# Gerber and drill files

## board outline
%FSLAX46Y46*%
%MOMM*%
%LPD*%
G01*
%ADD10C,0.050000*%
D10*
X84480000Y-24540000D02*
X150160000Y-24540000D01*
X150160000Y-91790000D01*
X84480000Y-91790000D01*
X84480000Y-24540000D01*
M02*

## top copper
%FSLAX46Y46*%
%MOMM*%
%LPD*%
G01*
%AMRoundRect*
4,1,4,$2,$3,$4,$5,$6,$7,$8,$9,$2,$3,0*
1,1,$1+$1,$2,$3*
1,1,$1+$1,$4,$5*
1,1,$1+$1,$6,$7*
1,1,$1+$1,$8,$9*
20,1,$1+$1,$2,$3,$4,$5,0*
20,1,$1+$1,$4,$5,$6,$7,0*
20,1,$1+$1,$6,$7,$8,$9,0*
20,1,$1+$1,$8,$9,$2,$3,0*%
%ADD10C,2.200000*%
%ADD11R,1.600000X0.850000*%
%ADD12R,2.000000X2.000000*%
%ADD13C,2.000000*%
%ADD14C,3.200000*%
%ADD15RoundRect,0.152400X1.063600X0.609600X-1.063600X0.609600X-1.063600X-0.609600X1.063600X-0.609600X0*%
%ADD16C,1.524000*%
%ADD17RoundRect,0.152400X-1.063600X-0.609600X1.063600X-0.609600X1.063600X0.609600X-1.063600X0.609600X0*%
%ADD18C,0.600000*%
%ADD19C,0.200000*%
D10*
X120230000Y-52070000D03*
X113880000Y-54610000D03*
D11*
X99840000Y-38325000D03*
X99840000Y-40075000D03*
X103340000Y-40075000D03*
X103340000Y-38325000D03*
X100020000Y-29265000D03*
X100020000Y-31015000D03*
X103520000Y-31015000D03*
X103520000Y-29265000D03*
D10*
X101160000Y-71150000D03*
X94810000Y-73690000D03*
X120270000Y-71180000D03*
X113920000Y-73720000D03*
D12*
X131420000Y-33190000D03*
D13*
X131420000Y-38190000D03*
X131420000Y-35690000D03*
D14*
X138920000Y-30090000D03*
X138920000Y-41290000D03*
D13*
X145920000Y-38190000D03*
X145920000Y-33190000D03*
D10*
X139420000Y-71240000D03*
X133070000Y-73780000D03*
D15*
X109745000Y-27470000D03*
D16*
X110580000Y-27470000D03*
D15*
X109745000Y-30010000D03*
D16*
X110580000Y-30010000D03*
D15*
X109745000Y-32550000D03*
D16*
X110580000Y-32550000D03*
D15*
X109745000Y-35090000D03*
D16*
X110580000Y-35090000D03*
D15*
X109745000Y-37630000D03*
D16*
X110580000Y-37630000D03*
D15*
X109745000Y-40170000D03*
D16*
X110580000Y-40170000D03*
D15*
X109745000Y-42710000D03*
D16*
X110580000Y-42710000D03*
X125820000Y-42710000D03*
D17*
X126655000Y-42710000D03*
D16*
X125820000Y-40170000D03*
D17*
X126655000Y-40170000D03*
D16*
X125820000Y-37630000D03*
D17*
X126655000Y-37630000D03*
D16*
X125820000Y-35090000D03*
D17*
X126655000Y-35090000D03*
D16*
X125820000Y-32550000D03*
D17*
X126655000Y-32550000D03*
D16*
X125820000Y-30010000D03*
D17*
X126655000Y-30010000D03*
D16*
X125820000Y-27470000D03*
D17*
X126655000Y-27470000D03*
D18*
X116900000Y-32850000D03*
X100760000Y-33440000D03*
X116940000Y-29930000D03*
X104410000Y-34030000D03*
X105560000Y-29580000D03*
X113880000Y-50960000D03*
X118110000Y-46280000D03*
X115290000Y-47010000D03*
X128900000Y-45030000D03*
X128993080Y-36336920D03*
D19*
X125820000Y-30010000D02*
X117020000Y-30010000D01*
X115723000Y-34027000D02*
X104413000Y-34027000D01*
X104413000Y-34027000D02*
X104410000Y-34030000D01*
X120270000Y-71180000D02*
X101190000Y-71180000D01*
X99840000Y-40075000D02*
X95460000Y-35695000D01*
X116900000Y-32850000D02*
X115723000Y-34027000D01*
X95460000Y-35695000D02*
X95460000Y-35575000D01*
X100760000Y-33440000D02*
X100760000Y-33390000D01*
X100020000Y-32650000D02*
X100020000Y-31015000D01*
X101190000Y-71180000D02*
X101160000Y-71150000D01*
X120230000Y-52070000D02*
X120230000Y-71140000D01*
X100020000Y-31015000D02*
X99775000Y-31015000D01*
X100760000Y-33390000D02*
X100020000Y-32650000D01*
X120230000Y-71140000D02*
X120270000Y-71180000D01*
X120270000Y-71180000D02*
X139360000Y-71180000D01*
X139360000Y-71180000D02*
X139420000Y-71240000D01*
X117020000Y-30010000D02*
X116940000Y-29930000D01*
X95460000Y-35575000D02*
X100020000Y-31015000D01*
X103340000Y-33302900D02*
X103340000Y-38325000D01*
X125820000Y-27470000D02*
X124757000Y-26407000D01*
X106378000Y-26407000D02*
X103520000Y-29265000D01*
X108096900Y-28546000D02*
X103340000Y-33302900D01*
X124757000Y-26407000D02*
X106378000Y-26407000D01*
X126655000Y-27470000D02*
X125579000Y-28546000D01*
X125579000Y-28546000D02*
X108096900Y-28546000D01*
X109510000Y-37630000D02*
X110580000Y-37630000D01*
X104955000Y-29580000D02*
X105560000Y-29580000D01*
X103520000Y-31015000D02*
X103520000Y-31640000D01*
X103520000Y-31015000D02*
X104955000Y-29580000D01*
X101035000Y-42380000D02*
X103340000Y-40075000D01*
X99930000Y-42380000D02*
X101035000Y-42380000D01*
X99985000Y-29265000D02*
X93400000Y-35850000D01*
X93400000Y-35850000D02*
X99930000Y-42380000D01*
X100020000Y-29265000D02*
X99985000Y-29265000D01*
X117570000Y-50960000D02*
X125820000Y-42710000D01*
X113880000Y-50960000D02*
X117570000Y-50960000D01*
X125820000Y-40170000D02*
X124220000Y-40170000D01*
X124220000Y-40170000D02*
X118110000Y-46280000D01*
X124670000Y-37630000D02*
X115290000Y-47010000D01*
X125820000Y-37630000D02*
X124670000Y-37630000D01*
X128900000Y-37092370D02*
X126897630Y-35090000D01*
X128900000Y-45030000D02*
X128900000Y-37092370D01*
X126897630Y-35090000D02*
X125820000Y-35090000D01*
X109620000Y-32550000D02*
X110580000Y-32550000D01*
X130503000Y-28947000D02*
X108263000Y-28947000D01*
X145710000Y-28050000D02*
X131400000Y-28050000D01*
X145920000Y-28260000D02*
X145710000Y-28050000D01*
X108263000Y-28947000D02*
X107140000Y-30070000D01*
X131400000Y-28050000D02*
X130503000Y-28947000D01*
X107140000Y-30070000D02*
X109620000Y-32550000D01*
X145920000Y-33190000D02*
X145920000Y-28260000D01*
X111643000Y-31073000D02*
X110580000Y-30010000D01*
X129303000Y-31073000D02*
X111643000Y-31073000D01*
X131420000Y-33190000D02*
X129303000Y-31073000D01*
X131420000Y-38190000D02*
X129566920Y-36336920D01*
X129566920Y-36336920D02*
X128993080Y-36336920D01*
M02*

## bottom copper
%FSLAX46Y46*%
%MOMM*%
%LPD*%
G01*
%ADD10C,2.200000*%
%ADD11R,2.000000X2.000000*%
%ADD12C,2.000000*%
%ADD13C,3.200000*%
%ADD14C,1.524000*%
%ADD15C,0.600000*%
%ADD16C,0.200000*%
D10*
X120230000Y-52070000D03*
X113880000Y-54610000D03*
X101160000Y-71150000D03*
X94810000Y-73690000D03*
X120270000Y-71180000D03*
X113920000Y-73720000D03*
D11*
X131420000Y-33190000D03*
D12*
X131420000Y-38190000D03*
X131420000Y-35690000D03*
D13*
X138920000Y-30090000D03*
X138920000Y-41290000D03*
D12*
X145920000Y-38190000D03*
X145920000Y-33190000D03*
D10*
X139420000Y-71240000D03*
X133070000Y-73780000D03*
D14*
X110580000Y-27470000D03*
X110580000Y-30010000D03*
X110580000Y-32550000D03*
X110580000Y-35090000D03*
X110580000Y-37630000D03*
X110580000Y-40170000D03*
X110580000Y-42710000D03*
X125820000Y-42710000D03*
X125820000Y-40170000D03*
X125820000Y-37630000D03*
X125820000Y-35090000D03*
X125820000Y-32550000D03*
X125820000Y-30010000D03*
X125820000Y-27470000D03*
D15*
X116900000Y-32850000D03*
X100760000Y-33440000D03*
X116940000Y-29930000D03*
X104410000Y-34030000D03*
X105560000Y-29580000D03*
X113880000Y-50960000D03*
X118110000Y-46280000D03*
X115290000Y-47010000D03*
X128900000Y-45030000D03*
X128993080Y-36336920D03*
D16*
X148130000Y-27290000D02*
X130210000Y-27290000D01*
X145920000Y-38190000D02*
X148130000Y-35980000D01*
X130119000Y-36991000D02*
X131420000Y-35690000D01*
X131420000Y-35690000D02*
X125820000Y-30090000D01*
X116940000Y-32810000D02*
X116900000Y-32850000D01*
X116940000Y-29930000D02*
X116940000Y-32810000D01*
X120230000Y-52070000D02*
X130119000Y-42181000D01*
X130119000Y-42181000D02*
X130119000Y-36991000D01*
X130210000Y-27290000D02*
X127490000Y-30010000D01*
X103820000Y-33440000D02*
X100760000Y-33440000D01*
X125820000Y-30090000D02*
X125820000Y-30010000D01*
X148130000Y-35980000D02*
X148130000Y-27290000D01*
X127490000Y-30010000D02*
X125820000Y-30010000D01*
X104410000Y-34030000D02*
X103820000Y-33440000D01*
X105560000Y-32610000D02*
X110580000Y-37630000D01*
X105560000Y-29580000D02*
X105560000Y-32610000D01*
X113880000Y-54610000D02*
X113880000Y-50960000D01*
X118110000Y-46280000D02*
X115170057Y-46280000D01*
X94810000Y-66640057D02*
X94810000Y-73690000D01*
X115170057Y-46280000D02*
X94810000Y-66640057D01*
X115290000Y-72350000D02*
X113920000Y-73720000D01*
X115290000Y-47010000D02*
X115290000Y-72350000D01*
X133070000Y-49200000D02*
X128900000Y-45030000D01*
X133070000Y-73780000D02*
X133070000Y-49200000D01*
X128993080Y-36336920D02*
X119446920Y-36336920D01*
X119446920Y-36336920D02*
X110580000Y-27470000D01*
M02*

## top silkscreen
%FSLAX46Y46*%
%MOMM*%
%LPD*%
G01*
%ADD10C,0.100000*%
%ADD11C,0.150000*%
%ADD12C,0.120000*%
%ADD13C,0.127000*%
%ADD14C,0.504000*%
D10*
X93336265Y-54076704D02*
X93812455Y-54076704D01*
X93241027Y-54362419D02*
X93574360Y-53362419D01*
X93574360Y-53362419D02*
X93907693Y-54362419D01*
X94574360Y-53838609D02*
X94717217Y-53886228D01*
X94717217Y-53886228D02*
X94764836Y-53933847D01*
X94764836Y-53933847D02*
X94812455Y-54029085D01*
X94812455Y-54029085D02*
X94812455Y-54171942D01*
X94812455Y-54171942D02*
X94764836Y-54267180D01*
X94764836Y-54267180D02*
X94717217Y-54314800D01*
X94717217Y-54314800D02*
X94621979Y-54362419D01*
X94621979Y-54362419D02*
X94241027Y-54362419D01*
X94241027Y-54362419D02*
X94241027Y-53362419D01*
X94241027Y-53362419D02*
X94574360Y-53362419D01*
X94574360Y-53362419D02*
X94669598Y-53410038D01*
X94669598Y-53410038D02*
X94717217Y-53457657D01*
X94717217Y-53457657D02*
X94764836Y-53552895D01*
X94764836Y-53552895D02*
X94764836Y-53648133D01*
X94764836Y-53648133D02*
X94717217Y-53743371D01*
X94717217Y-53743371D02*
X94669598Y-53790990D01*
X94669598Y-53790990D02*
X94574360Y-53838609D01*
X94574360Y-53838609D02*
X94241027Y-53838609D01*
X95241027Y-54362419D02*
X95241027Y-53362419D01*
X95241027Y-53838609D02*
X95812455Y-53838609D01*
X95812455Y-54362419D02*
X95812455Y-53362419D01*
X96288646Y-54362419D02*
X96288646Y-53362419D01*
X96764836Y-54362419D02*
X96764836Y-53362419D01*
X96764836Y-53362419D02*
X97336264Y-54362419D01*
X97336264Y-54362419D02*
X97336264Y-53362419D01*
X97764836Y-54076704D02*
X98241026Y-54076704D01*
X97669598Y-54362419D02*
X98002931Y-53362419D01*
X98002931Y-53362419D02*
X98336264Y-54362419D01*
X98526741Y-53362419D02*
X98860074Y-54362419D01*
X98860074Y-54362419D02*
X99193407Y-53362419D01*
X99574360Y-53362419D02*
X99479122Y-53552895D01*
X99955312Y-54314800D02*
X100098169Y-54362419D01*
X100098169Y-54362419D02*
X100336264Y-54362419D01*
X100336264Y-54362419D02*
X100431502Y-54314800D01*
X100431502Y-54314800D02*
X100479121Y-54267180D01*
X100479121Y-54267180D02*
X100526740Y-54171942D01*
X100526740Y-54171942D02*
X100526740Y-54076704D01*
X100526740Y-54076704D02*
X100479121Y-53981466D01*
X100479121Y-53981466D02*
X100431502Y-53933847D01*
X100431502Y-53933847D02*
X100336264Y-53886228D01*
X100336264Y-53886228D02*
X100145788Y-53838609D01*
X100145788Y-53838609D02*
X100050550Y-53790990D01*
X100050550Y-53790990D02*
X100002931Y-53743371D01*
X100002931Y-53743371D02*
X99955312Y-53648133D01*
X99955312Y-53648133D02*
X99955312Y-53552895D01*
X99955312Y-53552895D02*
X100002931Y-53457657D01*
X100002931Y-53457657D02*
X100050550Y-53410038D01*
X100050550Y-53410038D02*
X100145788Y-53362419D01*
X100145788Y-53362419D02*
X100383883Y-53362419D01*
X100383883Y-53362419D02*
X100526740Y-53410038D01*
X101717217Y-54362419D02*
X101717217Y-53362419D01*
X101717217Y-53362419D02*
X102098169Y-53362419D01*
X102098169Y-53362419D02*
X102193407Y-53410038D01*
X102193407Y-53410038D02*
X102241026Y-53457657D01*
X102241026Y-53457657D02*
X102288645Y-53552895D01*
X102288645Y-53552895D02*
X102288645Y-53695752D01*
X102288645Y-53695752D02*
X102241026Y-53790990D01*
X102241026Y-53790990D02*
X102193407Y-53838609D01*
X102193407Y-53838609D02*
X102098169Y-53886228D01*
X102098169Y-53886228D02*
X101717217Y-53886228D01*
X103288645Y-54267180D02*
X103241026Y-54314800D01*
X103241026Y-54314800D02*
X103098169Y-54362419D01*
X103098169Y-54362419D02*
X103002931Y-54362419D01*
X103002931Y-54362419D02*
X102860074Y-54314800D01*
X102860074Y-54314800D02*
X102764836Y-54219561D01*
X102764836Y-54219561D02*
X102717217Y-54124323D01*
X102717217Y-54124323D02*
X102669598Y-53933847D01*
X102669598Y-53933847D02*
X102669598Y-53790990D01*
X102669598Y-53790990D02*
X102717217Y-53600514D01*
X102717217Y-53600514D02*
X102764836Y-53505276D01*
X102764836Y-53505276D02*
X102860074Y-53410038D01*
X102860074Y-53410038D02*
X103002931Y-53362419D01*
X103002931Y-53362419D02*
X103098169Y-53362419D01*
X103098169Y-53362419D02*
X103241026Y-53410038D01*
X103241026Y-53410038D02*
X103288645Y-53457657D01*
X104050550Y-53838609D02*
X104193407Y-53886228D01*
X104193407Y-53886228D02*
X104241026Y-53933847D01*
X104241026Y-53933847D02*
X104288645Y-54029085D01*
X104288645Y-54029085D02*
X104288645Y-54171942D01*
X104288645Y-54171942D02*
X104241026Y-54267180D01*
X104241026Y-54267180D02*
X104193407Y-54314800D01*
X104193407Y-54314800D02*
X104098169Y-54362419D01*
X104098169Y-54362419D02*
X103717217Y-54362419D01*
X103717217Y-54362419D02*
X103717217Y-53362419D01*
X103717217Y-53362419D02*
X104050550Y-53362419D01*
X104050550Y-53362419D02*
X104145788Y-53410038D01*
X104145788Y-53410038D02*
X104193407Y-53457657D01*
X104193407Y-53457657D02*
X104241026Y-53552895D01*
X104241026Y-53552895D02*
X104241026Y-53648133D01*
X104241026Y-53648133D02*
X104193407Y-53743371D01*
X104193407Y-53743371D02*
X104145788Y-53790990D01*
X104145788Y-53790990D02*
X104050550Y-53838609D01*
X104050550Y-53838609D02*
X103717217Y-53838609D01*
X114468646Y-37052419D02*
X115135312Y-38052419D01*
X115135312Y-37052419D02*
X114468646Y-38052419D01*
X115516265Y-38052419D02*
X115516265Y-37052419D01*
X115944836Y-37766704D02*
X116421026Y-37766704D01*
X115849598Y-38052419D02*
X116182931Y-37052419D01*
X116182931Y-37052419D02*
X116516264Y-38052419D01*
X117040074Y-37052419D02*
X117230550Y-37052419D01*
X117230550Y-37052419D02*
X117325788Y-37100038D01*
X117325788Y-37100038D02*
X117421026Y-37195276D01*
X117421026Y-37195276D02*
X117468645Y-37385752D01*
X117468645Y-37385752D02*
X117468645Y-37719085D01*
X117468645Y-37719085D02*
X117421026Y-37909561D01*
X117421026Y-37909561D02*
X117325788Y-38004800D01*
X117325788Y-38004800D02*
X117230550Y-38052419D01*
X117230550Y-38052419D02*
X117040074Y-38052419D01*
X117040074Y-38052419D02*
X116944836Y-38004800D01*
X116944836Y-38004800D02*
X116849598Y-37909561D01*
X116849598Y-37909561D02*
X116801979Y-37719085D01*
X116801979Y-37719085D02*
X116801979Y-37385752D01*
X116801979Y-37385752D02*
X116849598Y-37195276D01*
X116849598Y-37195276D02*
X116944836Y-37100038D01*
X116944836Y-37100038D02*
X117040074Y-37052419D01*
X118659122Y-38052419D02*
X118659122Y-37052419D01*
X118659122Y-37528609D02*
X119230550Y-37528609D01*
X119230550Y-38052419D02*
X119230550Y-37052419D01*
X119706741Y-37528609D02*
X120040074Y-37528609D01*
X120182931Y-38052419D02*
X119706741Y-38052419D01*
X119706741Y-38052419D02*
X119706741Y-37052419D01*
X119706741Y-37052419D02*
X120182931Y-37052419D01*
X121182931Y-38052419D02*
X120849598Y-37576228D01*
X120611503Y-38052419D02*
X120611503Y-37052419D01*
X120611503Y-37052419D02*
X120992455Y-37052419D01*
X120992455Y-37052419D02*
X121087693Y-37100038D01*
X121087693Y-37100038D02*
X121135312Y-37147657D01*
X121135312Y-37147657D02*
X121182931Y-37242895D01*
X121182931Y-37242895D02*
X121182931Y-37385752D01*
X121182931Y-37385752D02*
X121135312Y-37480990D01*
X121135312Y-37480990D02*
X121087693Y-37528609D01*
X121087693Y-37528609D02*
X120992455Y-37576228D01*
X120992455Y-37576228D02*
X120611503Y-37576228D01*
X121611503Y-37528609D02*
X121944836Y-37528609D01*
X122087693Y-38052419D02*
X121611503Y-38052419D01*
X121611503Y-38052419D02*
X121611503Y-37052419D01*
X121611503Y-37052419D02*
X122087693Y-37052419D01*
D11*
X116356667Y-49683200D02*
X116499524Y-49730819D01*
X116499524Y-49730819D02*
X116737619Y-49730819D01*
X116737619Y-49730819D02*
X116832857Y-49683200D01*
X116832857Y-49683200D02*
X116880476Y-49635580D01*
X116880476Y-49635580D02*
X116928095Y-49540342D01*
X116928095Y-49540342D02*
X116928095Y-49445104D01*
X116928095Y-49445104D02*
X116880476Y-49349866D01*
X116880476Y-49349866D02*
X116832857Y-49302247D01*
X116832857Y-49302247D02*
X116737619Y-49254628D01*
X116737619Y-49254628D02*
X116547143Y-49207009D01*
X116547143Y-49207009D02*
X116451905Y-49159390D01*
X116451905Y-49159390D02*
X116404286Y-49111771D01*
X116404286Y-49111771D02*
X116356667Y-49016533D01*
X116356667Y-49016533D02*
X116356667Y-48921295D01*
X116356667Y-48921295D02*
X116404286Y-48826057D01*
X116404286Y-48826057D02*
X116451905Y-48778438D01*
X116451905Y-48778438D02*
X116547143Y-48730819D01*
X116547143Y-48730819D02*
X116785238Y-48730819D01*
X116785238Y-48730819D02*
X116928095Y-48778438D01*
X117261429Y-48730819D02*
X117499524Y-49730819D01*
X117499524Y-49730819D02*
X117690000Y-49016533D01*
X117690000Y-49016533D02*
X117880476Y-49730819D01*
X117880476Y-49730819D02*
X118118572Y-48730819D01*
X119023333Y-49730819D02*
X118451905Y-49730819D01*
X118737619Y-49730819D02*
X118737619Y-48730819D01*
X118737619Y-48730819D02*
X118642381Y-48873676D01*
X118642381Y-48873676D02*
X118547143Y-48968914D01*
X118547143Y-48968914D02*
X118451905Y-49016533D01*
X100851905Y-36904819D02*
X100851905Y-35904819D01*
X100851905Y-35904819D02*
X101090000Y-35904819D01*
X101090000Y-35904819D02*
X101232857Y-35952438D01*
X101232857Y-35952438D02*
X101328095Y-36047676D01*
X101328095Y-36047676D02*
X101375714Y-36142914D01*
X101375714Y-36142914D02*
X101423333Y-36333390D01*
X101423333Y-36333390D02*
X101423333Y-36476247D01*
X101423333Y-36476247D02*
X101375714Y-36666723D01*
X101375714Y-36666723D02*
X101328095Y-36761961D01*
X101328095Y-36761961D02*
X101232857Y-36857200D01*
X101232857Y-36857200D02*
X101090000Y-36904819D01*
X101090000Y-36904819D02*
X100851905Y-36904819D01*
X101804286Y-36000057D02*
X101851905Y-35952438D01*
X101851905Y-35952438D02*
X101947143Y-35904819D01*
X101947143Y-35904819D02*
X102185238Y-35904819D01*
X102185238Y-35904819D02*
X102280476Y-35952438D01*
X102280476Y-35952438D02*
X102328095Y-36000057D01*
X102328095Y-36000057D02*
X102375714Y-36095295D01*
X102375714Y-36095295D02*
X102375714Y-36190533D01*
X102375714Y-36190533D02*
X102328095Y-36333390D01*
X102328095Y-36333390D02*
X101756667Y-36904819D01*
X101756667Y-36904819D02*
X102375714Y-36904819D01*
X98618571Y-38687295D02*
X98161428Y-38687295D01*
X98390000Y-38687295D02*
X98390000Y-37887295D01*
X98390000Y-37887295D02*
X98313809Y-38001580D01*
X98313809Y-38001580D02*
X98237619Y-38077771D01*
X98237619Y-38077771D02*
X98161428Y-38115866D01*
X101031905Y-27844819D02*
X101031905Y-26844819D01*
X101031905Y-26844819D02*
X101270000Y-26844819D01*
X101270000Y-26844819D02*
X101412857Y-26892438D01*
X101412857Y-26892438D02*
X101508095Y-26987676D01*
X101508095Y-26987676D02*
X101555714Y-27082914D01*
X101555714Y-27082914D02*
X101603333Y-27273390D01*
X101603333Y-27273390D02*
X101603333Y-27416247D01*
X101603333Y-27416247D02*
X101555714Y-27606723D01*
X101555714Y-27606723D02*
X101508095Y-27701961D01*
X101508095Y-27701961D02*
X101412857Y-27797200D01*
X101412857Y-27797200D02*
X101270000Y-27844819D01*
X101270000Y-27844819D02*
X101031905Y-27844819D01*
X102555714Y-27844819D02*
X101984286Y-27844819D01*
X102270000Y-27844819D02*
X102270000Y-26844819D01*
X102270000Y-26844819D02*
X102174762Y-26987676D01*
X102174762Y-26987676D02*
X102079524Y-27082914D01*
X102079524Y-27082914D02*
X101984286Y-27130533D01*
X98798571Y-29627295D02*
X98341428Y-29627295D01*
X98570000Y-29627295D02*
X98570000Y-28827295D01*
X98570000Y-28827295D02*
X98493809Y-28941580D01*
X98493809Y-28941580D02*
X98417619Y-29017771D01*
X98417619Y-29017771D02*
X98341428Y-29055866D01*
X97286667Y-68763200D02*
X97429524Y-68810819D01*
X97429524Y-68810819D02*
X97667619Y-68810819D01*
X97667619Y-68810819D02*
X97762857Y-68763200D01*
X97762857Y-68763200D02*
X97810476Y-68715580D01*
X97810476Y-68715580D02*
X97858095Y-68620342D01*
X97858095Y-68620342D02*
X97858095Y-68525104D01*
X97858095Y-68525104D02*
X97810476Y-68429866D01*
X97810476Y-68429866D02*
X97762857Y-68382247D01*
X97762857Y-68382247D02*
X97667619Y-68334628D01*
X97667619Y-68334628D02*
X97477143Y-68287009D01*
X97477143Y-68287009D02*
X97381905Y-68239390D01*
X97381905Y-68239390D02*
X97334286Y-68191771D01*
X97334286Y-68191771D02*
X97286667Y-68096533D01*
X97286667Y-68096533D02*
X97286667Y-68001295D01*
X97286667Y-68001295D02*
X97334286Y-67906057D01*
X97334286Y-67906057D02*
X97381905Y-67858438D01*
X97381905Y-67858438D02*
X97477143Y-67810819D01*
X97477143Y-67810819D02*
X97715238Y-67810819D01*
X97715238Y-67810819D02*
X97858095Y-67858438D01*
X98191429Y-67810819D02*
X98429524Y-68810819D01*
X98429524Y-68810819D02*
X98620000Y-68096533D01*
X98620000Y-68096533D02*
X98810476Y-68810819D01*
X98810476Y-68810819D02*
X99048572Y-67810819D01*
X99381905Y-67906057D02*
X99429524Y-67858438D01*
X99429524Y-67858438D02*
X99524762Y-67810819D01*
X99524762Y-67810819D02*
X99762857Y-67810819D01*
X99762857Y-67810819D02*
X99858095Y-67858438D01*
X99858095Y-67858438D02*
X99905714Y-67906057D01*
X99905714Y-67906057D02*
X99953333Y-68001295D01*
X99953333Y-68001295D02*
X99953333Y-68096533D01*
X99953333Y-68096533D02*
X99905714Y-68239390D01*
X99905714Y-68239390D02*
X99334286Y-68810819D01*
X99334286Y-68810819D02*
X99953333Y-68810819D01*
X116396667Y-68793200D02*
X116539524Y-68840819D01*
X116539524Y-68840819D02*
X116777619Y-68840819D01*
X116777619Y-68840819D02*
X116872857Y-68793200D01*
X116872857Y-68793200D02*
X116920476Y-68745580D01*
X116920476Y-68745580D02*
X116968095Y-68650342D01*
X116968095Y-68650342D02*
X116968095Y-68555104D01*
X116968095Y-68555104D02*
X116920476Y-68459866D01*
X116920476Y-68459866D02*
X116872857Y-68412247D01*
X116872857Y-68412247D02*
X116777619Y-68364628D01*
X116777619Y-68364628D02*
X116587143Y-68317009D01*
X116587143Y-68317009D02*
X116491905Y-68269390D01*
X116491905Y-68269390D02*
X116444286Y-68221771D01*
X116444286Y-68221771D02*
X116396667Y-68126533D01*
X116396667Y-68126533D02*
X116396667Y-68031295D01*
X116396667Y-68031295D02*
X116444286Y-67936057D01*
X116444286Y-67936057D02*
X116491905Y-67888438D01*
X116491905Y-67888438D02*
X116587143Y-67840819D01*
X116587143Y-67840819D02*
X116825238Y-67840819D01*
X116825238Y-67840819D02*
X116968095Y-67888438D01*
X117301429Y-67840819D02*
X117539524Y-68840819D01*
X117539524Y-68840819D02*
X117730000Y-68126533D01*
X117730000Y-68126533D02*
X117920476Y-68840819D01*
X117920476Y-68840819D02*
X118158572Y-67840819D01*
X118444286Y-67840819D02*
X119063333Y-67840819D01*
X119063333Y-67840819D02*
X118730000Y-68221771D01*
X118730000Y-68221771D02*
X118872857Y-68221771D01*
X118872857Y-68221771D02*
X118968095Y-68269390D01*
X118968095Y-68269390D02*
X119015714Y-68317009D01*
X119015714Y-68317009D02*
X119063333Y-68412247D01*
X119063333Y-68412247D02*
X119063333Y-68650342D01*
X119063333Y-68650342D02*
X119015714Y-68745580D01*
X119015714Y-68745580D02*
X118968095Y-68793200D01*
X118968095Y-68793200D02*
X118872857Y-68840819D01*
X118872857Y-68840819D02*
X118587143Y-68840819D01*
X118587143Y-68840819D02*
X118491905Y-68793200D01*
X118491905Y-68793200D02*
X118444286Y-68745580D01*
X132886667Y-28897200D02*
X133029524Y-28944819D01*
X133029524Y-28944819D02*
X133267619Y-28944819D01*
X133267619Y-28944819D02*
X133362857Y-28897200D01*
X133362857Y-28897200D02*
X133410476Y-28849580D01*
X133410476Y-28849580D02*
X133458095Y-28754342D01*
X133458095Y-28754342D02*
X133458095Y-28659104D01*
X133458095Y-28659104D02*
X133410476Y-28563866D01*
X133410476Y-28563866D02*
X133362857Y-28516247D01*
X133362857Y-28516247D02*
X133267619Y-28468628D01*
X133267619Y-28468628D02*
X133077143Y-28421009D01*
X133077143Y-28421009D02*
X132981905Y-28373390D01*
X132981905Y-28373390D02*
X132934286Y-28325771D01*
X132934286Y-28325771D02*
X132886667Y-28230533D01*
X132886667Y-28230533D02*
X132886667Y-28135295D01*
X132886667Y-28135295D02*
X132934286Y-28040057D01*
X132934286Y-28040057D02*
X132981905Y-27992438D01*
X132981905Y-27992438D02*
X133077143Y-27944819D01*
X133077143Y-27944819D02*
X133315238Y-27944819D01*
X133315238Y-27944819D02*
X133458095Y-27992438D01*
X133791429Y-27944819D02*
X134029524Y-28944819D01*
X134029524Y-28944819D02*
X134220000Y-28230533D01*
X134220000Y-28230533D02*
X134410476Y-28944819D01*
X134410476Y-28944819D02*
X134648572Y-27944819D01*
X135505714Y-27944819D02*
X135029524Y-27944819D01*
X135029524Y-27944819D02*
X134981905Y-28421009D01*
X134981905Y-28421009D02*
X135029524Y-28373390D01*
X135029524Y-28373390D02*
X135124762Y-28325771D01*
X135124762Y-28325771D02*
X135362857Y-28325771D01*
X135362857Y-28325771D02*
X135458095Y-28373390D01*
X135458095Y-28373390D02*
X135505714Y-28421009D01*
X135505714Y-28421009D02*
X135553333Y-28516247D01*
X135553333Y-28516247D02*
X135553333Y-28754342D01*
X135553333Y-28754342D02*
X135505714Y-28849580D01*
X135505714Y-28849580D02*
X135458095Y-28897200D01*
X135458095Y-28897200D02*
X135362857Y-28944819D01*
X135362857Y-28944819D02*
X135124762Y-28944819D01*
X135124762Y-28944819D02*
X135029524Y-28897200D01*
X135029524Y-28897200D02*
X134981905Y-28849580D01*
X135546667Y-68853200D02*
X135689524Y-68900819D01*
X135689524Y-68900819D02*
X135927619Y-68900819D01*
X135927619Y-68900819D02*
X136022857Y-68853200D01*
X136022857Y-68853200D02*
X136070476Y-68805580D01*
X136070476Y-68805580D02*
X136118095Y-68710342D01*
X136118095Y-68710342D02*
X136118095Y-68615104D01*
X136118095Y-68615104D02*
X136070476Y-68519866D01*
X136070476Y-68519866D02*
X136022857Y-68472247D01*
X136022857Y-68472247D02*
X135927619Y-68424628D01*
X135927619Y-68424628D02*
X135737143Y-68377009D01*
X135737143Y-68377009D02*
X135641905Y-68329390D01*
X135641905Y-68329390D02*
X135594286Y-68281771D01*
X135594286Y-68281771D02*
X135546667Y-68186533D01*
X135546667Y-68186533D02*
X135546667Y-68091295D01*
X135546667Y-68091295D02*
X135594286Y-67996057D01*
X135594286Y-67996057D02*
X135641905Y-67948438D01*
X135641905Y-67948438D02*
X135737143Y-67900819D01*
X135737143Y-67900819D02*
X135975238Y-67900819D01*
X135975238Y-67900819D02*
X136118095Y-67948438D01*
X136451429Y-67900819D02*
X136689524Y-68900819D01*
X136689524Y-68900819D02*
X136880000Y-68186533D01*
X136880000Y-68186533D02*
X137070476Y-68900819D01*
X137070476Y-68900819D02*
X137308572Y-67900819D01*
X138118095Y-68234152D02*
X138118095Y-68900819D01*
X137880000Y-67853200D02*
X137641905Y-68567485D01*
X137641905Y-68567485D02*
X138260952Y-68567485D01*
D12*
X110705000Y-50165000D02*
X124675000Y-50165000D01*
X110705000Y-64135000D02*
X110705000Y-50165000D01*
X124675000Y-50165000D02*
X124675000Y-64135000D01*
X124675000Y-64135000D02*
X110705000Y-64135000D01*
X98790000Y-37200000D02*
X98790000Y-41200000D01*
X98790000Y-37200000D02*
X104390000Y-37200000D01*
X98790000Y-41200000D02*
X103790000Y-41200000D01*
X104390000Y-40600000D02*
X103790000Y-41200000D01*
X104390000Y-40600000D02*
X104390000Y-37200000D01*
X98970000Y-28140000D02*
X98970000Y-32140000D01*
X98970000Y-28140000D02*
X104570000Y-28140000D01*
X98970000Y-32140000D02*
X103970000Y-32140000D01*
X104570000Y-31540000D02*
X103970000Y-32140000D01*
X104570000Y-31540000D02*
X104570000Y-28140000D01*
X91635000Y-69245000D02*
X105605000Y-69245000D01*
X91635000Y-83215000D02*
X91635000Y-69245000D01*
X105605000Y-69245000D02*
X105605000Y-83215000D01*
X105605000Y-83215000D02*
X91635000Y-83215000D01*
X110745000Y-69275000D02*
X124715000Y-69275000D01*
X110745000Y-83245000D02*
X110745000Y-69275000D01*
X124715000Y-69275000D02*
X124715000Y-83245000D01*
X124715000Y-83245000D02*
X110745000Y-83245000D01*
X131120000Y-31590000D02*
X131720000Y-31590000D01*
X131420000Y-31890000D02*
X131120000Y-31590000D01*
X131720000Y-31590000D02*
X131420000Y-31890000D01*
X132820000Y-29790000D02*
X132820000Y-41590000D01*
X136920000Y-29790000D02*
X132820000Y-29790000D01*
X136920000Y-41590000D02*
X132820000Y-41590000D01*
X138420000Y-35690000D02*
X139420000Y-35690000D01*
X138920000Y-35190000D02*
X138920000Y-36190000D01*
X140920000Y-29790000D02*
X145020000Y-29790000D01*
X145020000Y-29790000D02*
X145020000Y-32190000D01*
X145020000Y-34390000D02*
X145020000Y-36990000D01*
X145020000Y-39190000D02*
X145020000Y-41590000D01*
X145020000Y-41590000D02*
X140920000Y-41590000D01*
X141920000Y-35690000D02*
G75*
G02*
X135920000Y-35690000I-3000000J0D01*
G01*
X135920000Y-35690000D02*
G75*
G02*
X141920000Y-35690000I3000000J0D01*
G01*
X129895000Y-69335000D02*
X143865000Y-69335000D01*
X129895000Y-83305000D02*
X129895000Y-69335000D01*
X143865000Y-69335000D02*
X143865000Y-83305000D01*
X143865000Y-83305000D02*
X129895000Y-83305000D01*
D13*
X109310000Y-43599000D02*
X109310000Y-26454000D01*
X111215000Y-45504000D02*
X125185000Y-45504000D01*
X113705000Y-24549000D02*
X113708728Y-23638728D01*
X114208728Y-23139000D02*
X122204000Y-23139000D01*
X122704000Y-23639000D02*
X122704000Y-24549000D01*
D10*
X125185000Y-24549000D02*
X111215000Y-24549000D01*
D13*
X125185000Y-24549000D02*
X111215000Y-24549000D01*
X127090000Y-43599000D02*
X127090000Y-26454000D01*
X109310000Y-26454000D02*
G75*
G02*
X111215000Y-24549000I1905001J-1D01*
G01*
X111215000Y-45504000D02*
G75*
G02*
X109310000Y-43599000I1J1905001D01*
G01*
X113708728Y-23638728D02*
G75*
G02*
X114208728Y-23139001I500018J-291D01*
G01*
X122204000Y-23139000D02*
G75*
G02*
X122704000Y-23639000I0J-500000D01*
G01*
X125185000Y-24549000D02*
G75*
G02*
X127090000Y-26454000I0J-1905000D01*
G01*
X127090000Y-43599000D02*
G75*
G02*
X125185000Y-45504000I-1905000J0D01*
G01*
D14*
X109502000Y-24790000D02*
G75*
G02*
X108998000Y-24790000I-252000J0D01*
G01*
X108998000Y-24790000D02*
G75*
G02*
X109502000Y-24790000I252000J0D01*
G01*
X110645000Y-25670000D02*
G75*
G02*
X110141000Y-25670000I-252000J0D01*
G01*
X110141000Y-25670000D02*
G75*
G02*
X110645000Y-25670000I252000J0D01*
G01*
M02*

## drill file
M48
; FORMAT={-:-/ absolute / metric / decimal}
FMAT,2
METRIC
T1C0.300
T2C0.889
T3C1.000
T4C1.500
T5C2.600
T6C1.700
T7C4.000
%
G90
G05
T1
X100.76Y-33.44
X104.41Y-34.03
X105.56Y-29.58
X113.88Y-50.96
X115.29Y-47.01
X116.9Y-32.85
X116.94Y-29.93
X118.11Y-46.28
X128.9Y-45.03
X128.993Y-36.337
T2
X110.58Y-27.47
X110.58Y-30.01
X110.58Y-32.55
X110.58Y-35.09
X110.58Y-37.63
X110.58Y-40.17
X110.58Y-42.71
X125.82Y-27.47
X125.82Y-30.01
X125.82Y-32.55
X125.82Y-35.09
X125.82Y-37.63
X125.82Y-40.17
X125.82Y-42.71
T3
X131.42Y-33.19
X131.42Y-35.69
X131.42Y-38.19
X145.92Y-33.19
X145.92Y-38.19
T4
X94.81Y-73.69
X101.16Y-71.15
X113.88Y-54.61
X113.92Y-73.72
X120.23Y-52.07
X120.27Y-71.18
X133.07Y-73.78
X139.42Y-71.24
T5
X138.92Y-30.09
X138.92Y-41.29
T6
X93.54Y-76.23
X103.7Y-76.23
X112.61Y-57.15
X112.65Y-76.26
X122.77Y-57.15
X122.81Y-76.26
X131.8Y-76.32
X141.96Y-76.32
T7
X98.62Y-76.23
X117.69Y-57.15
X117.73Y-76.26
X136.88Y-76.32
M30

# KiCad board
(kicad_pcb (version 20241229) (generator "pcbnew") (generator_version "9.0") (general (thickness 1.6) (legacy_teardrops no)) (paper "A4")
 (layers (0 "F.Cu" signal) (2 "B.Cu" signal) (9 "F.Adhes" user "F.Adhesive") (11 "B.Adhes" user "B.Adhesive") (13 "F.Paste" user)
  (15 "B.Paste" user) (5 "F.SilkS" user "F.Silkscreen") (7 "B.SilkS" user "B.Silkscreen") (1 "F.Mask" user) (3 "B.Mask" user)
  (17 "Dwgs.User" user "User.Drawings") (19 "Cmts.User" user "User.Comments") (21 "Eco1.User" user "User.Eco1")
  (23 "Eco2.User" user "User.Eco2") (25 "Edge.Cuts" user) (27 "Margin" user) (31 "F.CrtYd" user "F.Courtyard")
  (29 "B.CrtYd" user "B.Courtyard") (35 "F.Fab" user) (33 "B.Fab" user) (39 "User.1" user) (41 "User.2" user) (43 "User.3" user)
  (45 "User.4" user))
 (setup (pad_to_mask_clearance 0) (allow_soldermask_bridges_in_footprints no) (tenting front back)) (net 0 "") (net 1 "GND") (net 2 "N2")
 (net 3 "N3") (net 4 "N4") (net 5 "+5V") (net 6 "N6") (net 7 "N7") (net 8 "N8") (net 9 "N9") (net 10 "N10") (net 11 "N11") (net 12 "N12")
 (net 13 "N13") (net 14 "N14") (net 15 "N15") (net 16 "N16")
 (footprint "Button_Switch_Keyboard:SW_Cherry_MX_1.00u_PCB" (layer "F.Cu") (at 120.23 52.07)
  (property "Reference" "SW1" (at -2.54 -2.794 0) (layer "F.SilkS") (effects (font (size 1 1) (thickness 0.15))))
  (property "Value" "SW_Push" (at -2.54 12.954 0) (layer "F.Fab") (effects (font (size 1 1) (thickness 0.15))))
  (fp_line (start -9.525 -1.905) (end 4.445 -1.905) (stroke (width 0.12) (type solid)) (layer "F.SilkS"))
  (fp_line (start -9.525 12.065) (end -9.525 -1.905) (stroke (width 0.12) (type solid)) (layer "F.SilkS"))
  (fp_line (start 4.445 -1.905) (end 4.445 12.065) (stroke (width 0.12) (type solid)) (layer "F.SilkS"))
  (fp_line (start 4.445 12.065) (end -9.525 12.065) (stroke (width 0.12) (type solid)) (layer "F.SilkS"))
  (pad "" np_thru_hole circle (at -7.62 5.08) (size 1.7 1.7) (drill 1.7) (layers "*.Cu" "*.Mask"))
  (pad "" np_thru_hole circle (at -2.54 5.08) (size 4 4) (drill 4) (layers "*.Cu" "*.Mask"))
  (pad "" np_thru_hole circle (at 2.54 5.08) (size 1.7 1.7) (drill 1.7) (layers "*.Cu" "*.Mask"))
  (pad "1" thru_hole circle (at 0 0) (size 2.2 2.2) (drill 1.5) (layers "*.Cu" "*.Mask") (remove_unused_layers no) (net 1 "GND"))
  (pad "2" thru_hole circle (at -6.35 2.54) (size 2.2 2.2) (drill 1.5) (layers "*.Cu" "*.Mask") (remove_unused_layers no) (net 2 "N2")))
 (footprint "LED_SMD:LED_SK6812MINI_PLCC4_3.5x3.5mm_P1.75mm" (layer "F.Cu") (at 101.59 39.2)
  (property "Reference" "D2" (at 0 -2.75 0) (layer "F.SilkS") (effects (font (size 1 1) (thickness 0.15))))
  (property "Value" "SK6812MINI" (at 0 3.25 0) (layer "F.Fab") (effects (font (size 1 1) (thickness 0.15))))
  (fp_line (start -2.8 -2) (end -2.8 2) (stroke (width 0.12) (type default)) (layer "F.SilkS"))
  (fp_line (start -2.8 -2) (end 2.8 -2) (stroke (width 0.12) (type solid)) (layer "F.SilkS"))
  (fp_line (start -2.8 2) (end 2.2 2) (stroke (width 0.12) (type solid)) (layer "F.SilkS"))
  (fp_line (start 2.8 1.4) (end 2.2 2) (stroke (width 0.12) (type default)) (layer "F.SilkS"))
  (fp_line (start 2.8 1.4) (end 2.8 -2) (stroke (width 0.12) (type solid)) (layer "F.SilkS"))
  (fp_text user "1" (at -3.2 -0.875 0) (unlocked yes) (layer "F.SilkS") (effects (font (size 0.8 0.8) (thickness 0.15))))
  (pad "1" smd rect (at -1.75 -0.875) (size 1.6 0.85) (layers "F.Cu" "F.Mask" "F.Paste") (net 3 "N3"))
  (pad "2" smd rect (at -1.75 0.875) (size 1.6 0.85) (layers "F.Cu" "F.Mask" "F.Paste") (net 1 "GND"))
  (pad "3" smd rect (at 1.75 0.875) (size 1.6 0.85) (layers "F.Cu" "F.Mask" "F.Paste") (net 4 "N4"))
  (pad "4" smd rect (at 1.75 -0.875) (size 1.6 0.85) (layers "F.Cu" "F.Mask" "F.Paste") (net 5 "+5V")))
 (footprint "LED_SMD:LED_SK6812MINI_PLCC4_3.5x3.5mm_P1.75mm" (layer "F.Cu") (at 101.77 30.14)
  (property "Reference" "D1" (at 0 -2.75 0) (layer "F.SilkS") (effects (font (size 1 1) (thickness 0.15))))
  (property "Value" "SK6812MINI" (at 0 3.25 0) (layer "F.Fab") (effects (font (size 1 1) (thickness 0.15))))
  (fp_line (start -2.8 -2) (end -2.8 2) (stroke (width 0.12) (type default)) (layer "F.SilkS"))
  (fp_line (start -2.8 -2) (end 2.8 -2) (stroke (width 0.12) (type solid)) (layer "F.SilkS"))
  (fp_line (start -2.8 2) (end 2.2 2) (stroke (width 0.12) (type solid)) (layer "F.SilkS"))
  (fp_line (start 2.8 1.4) (end 2.2 2) (stroke (width 0.12) (type default)) (layer "F.SilkS"))
  (fp_line (start 2.8 1.4) (end 2.8 -2) (stroke (width 0.12) (type solid)) (layer "F.SilkS"))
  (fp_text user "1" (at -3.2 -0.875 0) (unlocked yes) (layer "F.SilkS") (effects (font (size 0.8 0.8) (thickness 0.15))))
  (pad "1" smd rect (at -1.75 -0.875) (size 1.6 0.85) (layers "F.Cu" "F.Mask" "F.Paste") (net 4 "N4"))
  (pad "2" smd rect (at -1.75 0.875) (size 1.6 0.85) (layers "F.Cu" "F.Mask" "F.Paste") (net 1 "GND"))
  (pad "3" smd rect (at 1.75 0.875) (size 1.6 0.85) (layers "F.Cu" "F.Mask" "F.Paste") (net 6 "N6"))
  (pad "4" smd rect (at 1.75 -0.875) (size 1.6 0.85) (layers "F.Cu" "F.Mask" "F.Paste") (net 5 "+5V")))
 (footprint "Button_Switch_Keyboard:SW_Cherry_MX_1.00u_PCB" (layer "F.Cu") (at 101.16 71.15)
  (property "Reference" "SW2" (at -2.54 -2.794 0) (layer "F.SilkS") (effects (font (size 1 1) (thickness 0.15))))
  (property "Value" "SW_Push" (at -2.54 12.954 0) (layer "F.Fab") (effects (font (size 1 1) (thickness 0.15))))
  (fp_line (start -9.525 -1.905) (end 4.445 -1.905) (stroke (width 0.12) (type solid)) (layer "F.SilkS"))
  (fp_line (start -9.525 12.065) (end -9.525 -1.905) (stroke (width 0.12) (type solid)) (layer "F.SilkS"))
  (fp_line (start 4.445 -1.905) (end 4.445 12.065) (stroke (width 0.12) (type solid)) (layer "F.SilkS"))
  (fp_line (start 4.445 12.065) (end -9.525 12.065) (stroke (width 0.12) (type solid)) (layer "F.SilkS"))
  (pad "" np_thru_hole circle (at -7.62 5.08) (size 1.7 1.7) (drill 1.7) (layers "*.Cu" "*.Mask"))
  (pad "" np_thru_hole circle (at -2.54 5.08) (size 4 4) (drill 4) (layers "*.Cu" "*.Mask"))
  (pad "" np_thru_hole circle (at 2.54 5.08) (size 1.7 1.7) (drill 1.7) (layers "*.Cu" "*.Mask"))
  (pad "1" thru_hole circle (at 0 0) (size 2.2 2.2) (drill 1.5) (layers "*.Cu" "*.Mask") (remove_unused_layers no) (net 1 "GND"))
  (pad "2" thru_hole circle (at -6.35 2.54) (size 2.2 2.2) (drill 1.5) (layers "*.Cu" "*.Mask") (remove_unused_layers no) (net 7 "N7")))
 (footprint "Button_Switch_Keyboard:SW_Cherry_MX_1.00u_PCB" (layer "F.Cu") (at 120.27 71.18)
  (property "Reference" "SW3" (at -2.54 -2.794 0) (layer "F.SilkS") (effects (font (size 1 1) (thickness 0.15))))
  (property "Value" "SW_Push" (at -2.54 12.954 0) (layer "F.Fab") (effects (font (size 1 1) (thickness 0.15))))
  (fp_line (start -9.525 -1.905) (end 4.445 -1.905) (stroke (width 0.12) (type solid)) (layer "F.SilkS"))
  (fp_line (start -9.525 12.065) (end -9.525 -1.905) (stroke (width 0.12) (type solid)) (layer "F.SilkS"))
  (fp_line (start 4.445 -1.905) (end 4.445 12.065) (stroke (width 0.12) (type solid)) (layer "F.SilkS"))
  (fp_line (start 4.445 12.065) (end -9.525 12.065) (stroke (width 0.12) (type solid)) (layer "F.SilkS"))
  (pad "" np_thru_hole circle (at -7.62 5.08) (size 1.7 1.7) (drill 1.7) (layers "*.Cu" "*.Mask"))
  (pad "" np_thru_hole circle (at -2.54 5.08) (size 4 4) (drill 4) (layers "*.Cu" "*.Mask"))
  (pad "" np_thru_hole circle (at 2.54 5.08) (size 1.7 1.7) (drill 1.7) (layers "*.Cu" "*.Mask"))
  (pad "1" thru_hole circle (at 0 0) (size 2.2 2.2) (drill 1.5) (layers "*.Cu" "*.Mask") (remove_unused_layers no) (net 1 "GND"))
  (pad "2" thru_hole circle (at -6.35 2.54) (size 2.2 2.2) (drill 1.5) (layers "*.Cu" "*.Mask") (remove_unused_layers no) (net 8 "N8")))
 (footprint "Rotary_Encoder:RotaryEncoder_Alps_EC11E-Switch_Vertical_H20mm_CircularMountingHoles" (layer "F.Cu") (at 131.42 33.19)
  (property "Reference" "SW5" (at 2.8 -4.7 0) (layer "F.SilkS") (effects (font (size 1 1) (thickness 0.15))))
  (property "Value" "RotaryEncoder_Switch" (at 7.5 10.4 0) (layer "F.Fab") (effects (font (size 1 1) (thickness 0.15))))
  (fp_line (start -0.3 -1.6) (end 0.3 -1.6) (stroke (width 0.12) (type solid)) (layer "F.SilkS"))
  (fp_line (start 0 -1.3) (end -0.3 -1.6) (stroke (width 0.12) (type solid)) (layer "F.SilkS"))
  (fp_line (start 0.3 -1.6) (end 0 -1.3) (stroke (width 0.12) (type solid)) (layer "F.SilkS"))
  (fp_line (start 1.4 -3.4) (end 1.4 8.4) (stroke (width 0.12) (type solid)) (layer "F.SilkS"))
  (fp_line (start 5.5 -3.4) (end 1.4 -3.4) (stroke (width 0.12) (type solid)) (layer "F.SilkS"))
  (fp_line (start 5.5 8.4) (end 1.4 8.4) (stroke (width 0.12) (type solid)) (layer "F.SilkS"))
  (fp_line (start 7 2.5) (end 8 2.5) (stroke (width 0.12) (type solid)) (layer "F.SilkS"))
  (fp_line (start 7.5 2) (end 7.5 3) (stroke (width 0.12) (type solid)) (layer "F.SilkS"))
  (fp_line (start 9.5 -3.4) (end 13.6 -3.4) (stroke (width 0.12) (type solid)) (layer "F.SilkS"))
  (fp_line (start 13.6 -3.4) (end 13.6 -1) (stroke (width 0.12) (type solid)) (layer "F.SilkS"))
  (fp_line (start 13.6 1.2) (end 13.6 3.8) (stroke (width 0.12) (type solid)) (layer "F.SilkS"))
  (fp_line (start 13.6 6) (end 13.6 8.4) (stroke (width 0.12) (type solid)) (layer "F.SilkS"))
  (fp_line (start 13.6 8.4) (end 9.5 8.4) (stroke (width 0.12) (type solid)) (layer "F.SilkS"))
  (fp_circle (center 7.5 2.5) (end 10.5 2.5) (stroke (width 0.12) (type solid)) (fill no) (layer "F.SilkS"))
  (pad "A" thru_hole rect (at 0 0) (size 2 2) (drill 1) (layers "*.Cu" "*.Mask") (remove_unused_layers no) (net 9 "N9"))
  (pad "B" thru_hole circle (at 0 5) (size 2 2) (drill 1) (layers "*.Cu" "*.Mask") (remove_unused_layers no) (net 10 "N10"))
  (pad "C" thru_hole circle (at 0 2.5) (size 2 2) (drill 1) (layers "*.Cu" "*.Mask") (remove_unused_layers no) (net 1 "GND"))
  (pad "MP" thru_hole circle (at 7.5 -3.1) (size 3.2 3.2) (drill 2.6) (layers "*.Cu" "*.Mask") (remove_unused_layers no))
  (pad "MP" thru_hole circle (at 7.5 8.1) (size 3.2 3.2) (drill 2.6) (layers "*.Cu" "*.Mask") (remove_unused_layers no))
  (pad "S1" thru_hole circle (at 14.5 5) (size 2 2) (drill 1) (layers "*.Cu" "*.Mask") (remove_unused_layers no) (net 1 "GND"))
  (pad "S2" thru_hole circle (at 14.5 0) (size 2 2) (drill 1) (layers "*.Cu" "*.Mask") (remove_unused_layers no) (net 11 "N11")))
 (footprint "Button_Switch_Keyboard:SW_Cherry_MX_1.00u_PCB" (layer "F.Cu") (at 139.42 71.24)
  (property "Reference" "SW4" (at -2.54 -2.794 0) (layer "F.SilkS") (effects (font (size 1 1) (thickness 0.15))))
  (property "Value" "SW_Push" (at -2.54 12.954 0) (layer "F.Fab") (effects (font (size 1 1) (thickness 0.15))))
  (fp_line (start -9.525 -1.905) (end 4.445 -1.905) (stroke (width 0.12) (type solid)) (layer "F.SilkS"))
  (fp_line (start -9.525 12.065) (end -9.525 -1.905) (stroke (width 0.12) (type solid)) (layer "F.SilkS"))
  (fp_line (start 4.445 -1.905) (end 4.445 12.065) (stroke (width 0.12) (type solid)) (layer "F.SilkS"))
  (fp_line (start 4.445 12.065) (end -9.525 12.065) (stroke (width 0.12) (type solid)) (layer "F.SilkS"))
  (pad "" np_thru_hole circle (at -7.62 5.08) (size 1.7 1.7) (drill 1.7) (layers "*.Cu" "*.Mask"))
  (pad "" np_thru_hole circle (at -2.54 5.08) (size 4 4) (drill 4) (layers "*.Cu" "*.Mask"))
  (pad "" np_thru_hole circle (at 2.54 5.08) (size 1.7 1.7) (drill 1.7) (layers "*.Cu" "*.Mask"))
  (pad "1" thru_hole circle (at 0 0) (size 2.2 2.2) (drill 1.5) (layers "*.Cu" "*.Mask") (remove_unused_layers no) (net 1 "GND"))
  (pad "2" thru_hole circle (at -6.35 2.54) (size 2.2 2.2) (drill 1.5) (layers "*.Cu" "*.Mask") (remove_unused_layers no) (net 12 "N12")))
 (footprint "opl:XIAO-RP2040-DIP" (layer "F.Cu") (at 118.2 35.09)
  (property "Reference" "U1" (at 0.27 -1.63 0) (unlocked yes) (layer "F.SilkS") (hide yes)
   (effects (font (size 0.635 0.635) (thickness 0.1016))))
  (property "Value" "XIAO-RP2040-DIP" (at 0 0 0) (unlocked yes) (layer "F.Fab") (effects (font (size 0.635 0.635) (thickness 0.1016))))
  (fp_line (start -8.89 8.509) (end -8.89 -8.636) (stroke (width 0.127) (type solid)) (layer "F.SilkS"))
  (fp_line (start -6.985 10.414) (end 6.985 10.414) (stroke (width 0.127) (type solid)) (layer "F.SilkS"))
  (fp_line (start -4.495 -10.541) (end -4.491272 -11.451272) (stroke (width 0.127) (type solid)) (layer "F.SilkS"))
  (fp_line (start -3.991272 -11.951) (end 4.004 -11.951) (stroke (width 0.127) (type solid)) (layer "F.SilkS"))
  (fp_line (start 4.504 -11.451) (end 4.504 -10.541) (stroke (width 0.127) (type solid)) (layer "F.SilkS"))
  (fp_line (start 6.985 -10.541) (end -6.985 -10.541) (stroke (width 0.1) (type solid)) (layer "F.SilkS"))
  (fp_line (start 6.985 -10.541) (end -6.985 -10.541) (stroke (width 0.127) (type solid)) (layer "F.SilkS"))
  (fp_line (start 8.89 8.509) (end 8.89 -8.636) (stroke (width 0.127) (type solid)) (layer "F.SilkS"))
  (fp_arc (start -8.89 -8.636) (mid -8.332038 -9.983038) (end -6.985 -10.541) (stroke (width 0.127) (type solid)) (layer "F.SilkS"))
  (fp_arc (start -6.985 10.414) (mid -8.332038 9.856038) (end -8.89 8.509) (stroke (width 0.127) (type solid)) (layer "F.SilkS"))
  (fp_arc (start -4.491272 -11.451272) (mid -4.344728 -11.80464) (end -3.991272 -11.951) (stroke (width 0.127) (type default))
   (layer "F.SilkS"))
  (fp_arc (start 4.004 -11.951) (mid 4.357553 -11.804553) (end 4.504 -11.451) (stroke (width 0.127) (type default)) (layer "F.SilkS"))
  (fp_arc (start 6.985 -10.541) (mid 8.332038 -9.983038) (end 8.89 -8.636) (stroke (width 0.127) (type solid)) (layer "F.SilkS"))
  (fp_arc (start 8.89 8.509) (mid 8.332038 9.856038) (end 6.985 10.414) (stroke (width 0.127) (type solid)) (layer "F.SilkS"))
  (fp_circle (center -8.95 -10.3) (end -8.95 -10.554) (stroke (width 0.5) (type solid)) (fill yes) (layer "F.SilkS"))
  (fp_circle (center -7.807 -9.42) (end -7.807 -9.674) (stroke (width 0.5) (type solid)) (fill yes) (layer "F.SilkS"))
  (pad "1" smd roundrect (at -8.455 -7.62 180) (size 2.432 1.524) (layers "F.Cu" "F.Mask") (roundrect_rratio 0.1) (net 10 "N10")
   (thermal_bridge_angle 45))
  (pad "1" thru_hole circle (at -7.62 -7.62 180) (size 1.524 1.524) (drill 0.889) (layers "*.Cu" "*.Mask") (remove_unused_layers no)
   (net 10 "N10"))
  (pad "2" smd roundrect (at -8.455 -5.08 180) (size 2.432 1.524) (layers "F.Cu" "F.Mask") (roundrect_rratio 0.1) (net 9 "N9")
   (thermal_bridge_angle 45))
  (pad "2" thru_hole circle (at -7.62 -5.08 180) (size 1.524 1.524) (drill 0.889) (layers "*.Cu" "*.Mask") (remove_unused_layers no)
   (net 9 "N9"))
  (pad "3" smd roundrect (at -8.455 -2.54 180) (size 2.432 1.524) (layers "F.Cu" "F.Mask") (roundrect_rratio 0.1) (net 11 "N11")
   (thermal_bridge_angle 45))
  (pad "3" thru_hole circle (at -7.62 -2.54 180) (size 1.524 1.524) (drill 0.889) (layers "*.Cu" "*.Mask") (remove_unused_layers no)
   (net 11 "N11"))
  (pad "4" smd roundrect (at -8.455 0 180) (size 2.432 1.524) (layers "F.Cu" "F.Mask") (roundrect_rratio 0.1) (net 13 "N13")
   (thermal_bridge_angle 45))
  (pad "4" thru_hole circle (at -7.62 0 180) (size 1.524 1.524) (drill 0.889) (layers "*.Cu" "*.Mask") (remove_unused_layers no)
   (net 13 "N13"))
  (pad "5" smd roundrect (at -8.455 2.54 180) (size 2.432 1.524) (layers "F.Cu" "F.Mask") (roundrect_rratio 0.1) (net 6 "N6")
   (thermal_bridge_angle 45))
  (pad "5" thru_hole circle (at -7.62 2.54 180) (size 1.524 1.524) (drill 0.889) (layers "*.Cu" "*.Mask") (remove_unused_layers no)
   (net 6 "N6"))
  (pad "6" smd roundrect (at -8.455 5.08 180) (size 2.432 1.524) (layers "F.Cu" "F.Mask") (roundrect_rratio 0.1) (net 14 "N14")
   (thermal_bridge_angle 45))
  (pad "6" thru_hole circle (at -7.62 5.08 180) (size 1.524 1.524) (drill 0.889) (layers "*.Cu" "*.Mask") (remove_unused_layers no)
   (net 14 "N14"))
  (pad "7" smd roundrect (at -8.455 7.62 180) (size 2.432 1.524) (layers "F.Cu" "F.Mask") (roundrect_rratio 0.1) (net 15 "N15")
   (thermal_bridge_angle 45))
  (pad "7" thru_hole circle (at -7.62 7.62 180) (size 1.524 1.524) (drill 0.889) (layers "*.Cu" "*.Mask") (remove_unused_layers no)
   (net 15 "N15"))
  (pad "8" thru_hole circle (at 7.62 7.62) (size 1.524 1.524) (drill 0.889) (layers "*.Cu" "*.Mask") (remove_unused_layers no) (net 2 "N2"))
  (pad "8" smd roundrect (at 8.455 7.62) (size 2.432 1.524) (layers "F.Cu" "F.Mask") (roundrect_rratio 0.1) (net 2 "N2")
   (thermal_bridge_angle 45))
  (pad "9" thru_hole circle (at 7.62 5.08) (size 1.524 1.524) (drill 0.889) (layers "*.Cu" "*.Mask") (remove_unused_layers no) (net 7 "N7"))
  (pad "9" smd roundrect (at 8.455 5.08) (size 2.432 1.524) (layers "F.Cu" "F.Mask") (roundrect_rratio 0.1) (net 7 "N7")
   (thermal_bridge_angle 45))
  (pad "10" thru_hole circle (at 7.62 2.54) (size 1.524 1.524) (drill 0.889) (layers "*.Cu" "*.Mask") (remove_unused_layers no) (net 8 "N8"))
  (pad "10" smd roundrect (at 8.455 2.54) (size 2.432 1.524) (layers "F.Cu" "F.Mask") (roundrect_rratio 0.1) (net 8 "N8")
   (thermal_bridge_angle 45))
  (pad "11" thru_hole circle (at 7.62 0) (size 1.524 1.524) (drill 0.889) (layers "*.Cu" "*.Mask") (remove_unused_layers no) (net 12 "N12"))
  (pad "11" smd roundrect (at 8.455 0) (size 2.432 1.524) (layers "F.Cu" "F.Mask") (roundrect_rratio 0.1) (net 12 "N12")
   (thermal_bridge_angle 45))
  (pad "12" thru_hole circle (at 7.62 -2.54) (size 1.524 1.524) (drill 0.889) (layers "*.Cu" "*.Mask") (remove_unused_layers no)
   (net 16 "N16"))
  (pad "12" smd roundrect (at 8.455 -2.54) (size 2.432 1.524) (layers "F.Cu" "F.Mask") (roundrect_rratio 0.1) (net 16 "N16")
   (thermal_bridge_angle 45))
  (pad "13" thru_hole circle (at 7.62 -5.08) (size 1.524 1.524) (drill 0.889) (layers "*.Cu" "*.Mask") (remove_unused_layers no)
   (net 1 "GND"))
  (pad "13" smd roundrect (at 8.455 -5.08) (size 2.432 1.524) (layers "F.Cu" "F.Mask") (roundrect_rratio 0.1) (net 1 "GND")
   (thermal_bridge_angle 45))
  (pad "14" thru_hole circle (at 7.62 -7.62) (size 1.524 1.524) (drill 0.889) (layers "*.Cu" "*.Mask") (remove_unused_layers no)
   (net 5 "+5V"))
  (pad "14" smd roundrect (at 8.455 -7.62) (size 2.432 1.524) (layers "F.Cu" "F.Mask") (roundrect_rratio 0.1) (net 5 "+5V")
   (thermal_bridge_angle 45)))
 (gr_rect (start 84.48 24.54) (end 150.16 91.79) (stroke (width 0.05) (type default)) (fill no) (layer "Edge.Cuts"))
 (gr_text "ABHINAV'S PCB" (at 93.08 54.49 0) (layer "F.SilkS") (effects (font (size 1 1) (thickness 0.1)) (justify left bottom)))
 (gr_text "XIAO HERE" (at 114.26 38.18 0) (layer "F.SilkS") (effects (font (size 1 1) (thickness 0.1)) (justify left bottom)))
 (segment (start 125.82 30.01) (end 117.02 30.01) (width 0.2) (layer "F.Cu") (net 1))
 (segment (start 115.723 34.027) (end 104.413 34.027) (width 0.2) (layer "F.Cu") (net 1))
 (segment (start 104.413 34.027) (end 104.41 34.03) (width 0.2) (layer "F.Cu") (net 1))
 (segment (start 120.27 71.18) (end 101.19 71.18) (width 0.2) (layer "F.Cu") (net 1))
 (segment (start 99.84 40.075) (end 95.46 35.695) (width 0.2) (layer "F.Cu") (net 1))
 (segment (start 116.9 32.85) (end 115.723 34.027) (width 0.2) (layer "F.Cu") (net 1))
 (segment (start 95.46 35.695) (end 95.46 35.575) (width 0.2) (layer "F.Cu") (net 1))
 (segment (start 100.76 33.44) (end 100.76 33.39) (width 0.2) (layer "F.Cu") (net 1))
 (segment (start 100.02 32.65) (end 100.02 31.015) (width 0.2) (layer "F.Cu") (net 1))
 (segment (start 101.19 71.18) (end 101.16 71.15) (width 0.2) (layer "F.Cu") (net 1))
 (segment (start 120.23 52.07) (end 120.23 71.14) (width 0.2) (layer "F.Cu") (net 1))
 (segment (start 100.02 31.015) (end 99.775 31.015) (width 0.2) (layer "F.Cu") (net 1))
 (segment (start 100.76 33.39) (end 100.02 32.65) (width 0.2) (layer "F.Cu") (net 1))
 (segment (start 120.23 71.14) (end 120.27 71.18) (width 0.2) (layer "F.Cu") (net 1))
 (segment (start 120.27 71.18) (end 139.36 71.18) (width 0.2) (layer "F.Cu") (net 1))
 (segment (start 139.36 71.18) (end 139.42 71.24) (width 0.2) (layer "F.Cu") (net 1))
 (segment (start 117.02 30.01) (end 116.94 29.93) (width 0.2) (layer "F.Cu") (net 1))
 (segment (start 95.46 35.575) (end 100.02 31.015) (width 0.2) (layer "F.Cu") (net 1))
 (via (at 116.9 32.85) (size 0.6) (drill 0.3) (layers "F.Cu" "B.Cu") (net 1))
 (via (at 100.76 33.44) (size 0.6) (drill 0.3) (layers "F.Cu" "B.Cu") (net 1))
 (via (at 116.94 29.93) (size 0.6) (drill 0.3) (layers "F.Cu" "B.Cu") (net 1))
 (via (at 104.41 34.03) (size 0.6) (drill 0.3) (layers "F.Cu" "B.Cu") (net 1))
 (segment (start 148.13 27.29) (end 130.21 27.29) (width 0.2) (layer "B.Cu") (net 1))
 (segment (start 145.92 38.19) (end 148.13 35.98) (width 0.2) (layer "B.Cu") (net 1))
 (segment (start 130.119 36.991) (end 131.42 35.69) (width 0.2) (layer "B.Cu") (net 1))
 (segment (start 131.42 35.69) (end 125.82 30.09) (width 0.2) (layer "B.Cu") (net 1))
 (segment (start 116.94 32.81) (end 116.9 32.85) (width 0.2) (layer "B.Cu") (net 1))
 (segment (start 116.94 29.93) (end 116.94 32.81) (width 0.2) (layer "B.Cu") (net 1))
 (segment (start 120.23 52.07) (end 130.119 42.181) (width 0.2) (layer "B.Cu") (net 1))
 (segment (start 130.119 42.181) (end 130.119 36.991) (width 0.2) (layer "B.Cu") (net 1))
 (segment (start 130.21 27.29) (end 127.49 30.01) (width 0.2) (layer "B.Cu") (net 1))
 (segment (start 103.82 33.44) (end 100.76 33.44) (width 0.2) (layer "B.Cu") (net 1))
 (segment (start 125.82 30.09) (end 125.82 30.01) (width 0.2) (layer "B.Cu") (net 1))
 (segment (start 148.13 35.98) (end 148.13 27.29) (width 0.2) (layer "B.Cu") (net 1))
 (segment (start 127.49 30.01) (end 125.82 30.01) (width 0.2) (layer "B.Cu") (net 1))
 (segment (start 104.41 34.03) (end 103.82 33.44) (width 0.2) (layer "B.Cu") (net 1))
 (segment (start 103.34 33.3029) (end 103.34 38.325) (width 0.2) (layer "F.Cu") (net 5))
 (segment (start 125.82 27.47) (end 124.757 26.407) (width 0.2) (layer "F.Cu") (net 5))
 (segment (start 106.378 26.407) (end 103.52 29.265) (width 0.2) (layer "F.Cu") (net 5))
 (segment (start 108.0969 28.546) (end 103.34 33.3029) (width 0.2) (layer "F.Cu") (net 5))
 (segment (start 124.757 26.407) (end 106.378 26.407) (width 0.2) (layer "F.Cu") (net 5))
 (segment (start 126.655 27.47) (end 125.579 28.546) (width 0.2) (layer "F.Cu") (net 5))
 (segment (start 125.579 28.546) (end 108.0969 28.546) (width 0.2) (layer "F.Cu") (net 5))
 (segment (start 109.51 37.63) (end 110.58 37.63) (width 0.2) (layer "F.Cu") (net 6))
 (segment (start 104.955 29.58) (end 105.56 29.58) (width 0.2) (layer "F.Cu") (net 6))
 (segment (start 103.52 31.015) (end 103.52 31.64) (width 0.2) (layer "F.Cu") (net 6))
 (segment (start 103.52 31.015) (end 104.955 29.58) (width 0.2) (layer "F.Cu") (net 6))
 (via (at 105.56 29.58) (size 0.6) (drill 0.3) (layers "F.Cu" "B.Cu") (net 6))
 (segment (start 105.56 32.61) (end 110.58 37.63) (width 0.2) (layer "B.Cu") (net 6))
 (segment (start 105.56 29.58) (end 105.56 32.61) (width 0.2) (layer "B.Cu") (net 6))
 (segment (start 101.035 42.38) (end 103.34 40.075) (width 0.2) (layer "F.Cu") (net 4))
 (segment (start 99.93 42.38) (end 101.035 42.38) (width 0.2) (layer "F.Cu") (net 4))
 (segment (start 99.985 29.265) (end 93.4 35.85) (width 0.2) (layer "F.Cu") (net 4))
 (segment (start 93.4 35.85) (end 99.93 42.38) (width 0.2) (layer "F.Cu") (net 4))
 (segment (start 100.02 29.265) (end 99.985 29.265) (width 0.2) (layer "F.Cu") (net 4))
 (segment (start 117.57 50.96) (end 125.82 42.71) (width 0.2) (layer "F.Cu") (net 2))
 (segment (start 113.88 50.96) (end 117.57 50.96) (width 0.2) (layer "F.Cu") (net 2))
 (via (at 113.88 50.96) (size 0.6) (drill 0.3) (layers "F.Cu" "B.Cu") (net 2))
 (segment (start 113.88 54.61) (end 113.88 50.96) (width 0.2) (layer "B.Cu") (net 2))
 (segment (start 125.82 40.17) (end 124.22 40.17) (width 0.2) (layer "F.Cu") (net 7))
 (segment (start 124.22 40.17) (end 118.11 46.28) (width 0.2) (layer "F.Cu") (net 7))
 (via (at 118.11 46.28) (size 0.6) (drill 0.3) (layers "F.Cu" "B.Cu") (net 7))
 (segment (start 118.11 46.28) (end 115.170057 46.28) (width 0.2) (layer "B.Cu") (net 7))
 (segment (start 94.81 66.640057) (end 94.81 73.69) (width 0.2) (layer "B.Cu") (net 7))
 (segment (start 115.170057 46.28) (end 94.81 66.640057) (width 0.2) (layer "B.Cu") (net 7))
 (segment (start 124.67 37.63) (end 115.29 47.01) (width 0.2) (layer "F.Cu") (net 8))
 (segment (start 125.82 37.63) (end 124.67 37.63) (width 0.2) (layer "F.Cu") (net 8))
 (via (at 115.29 47.01) (size 0.6) (drill 0.3) (layers "F.Cu" "B.Cu") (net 8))
 (segment (start 115.29 72.35) (end 113.92 73.72) (width 0.2) (layer "B.Cu") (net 8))
 (segment (start 115.29 47.01) (end 115.29 72.35) (width 0.2) (layer "B.Cu") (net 8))
 (segment (start 128.9 37.09237) (end 126.89763 35.09) (width 0.2) (layer "F.Cu") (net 12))
 (segment (start 128.9 45.03) (end 128.9 37.09237) (width 0.2) (layer "F.Cu") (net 12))
 (segment (start 126.89763 35.09) (end 125.82 35.09) (width 0.2) (layer "F.Cu") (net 12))
 (via (at 128.9 45.03) (size 0.6) (drill 0.3) (layers "F.Cu" "B.Cu") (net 12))
 (segment (start 133.07 49.2) (end 128.9 45.03) (width 0.2) (layer "B.Cu") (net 12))
 (segment (start 133.07 73.78) (end 133.07 49.2) (width 0.2) (layer "B.Cu") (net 12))
 (segment (start 109.62 32.55) (end 110.58 32.55) (width 0.2) (layer "F.Cu") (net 11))
 (segment (start 130.503 28.947) (end 108.263 28.947) (width 0.2) (layer "F.Cu") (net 11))
 (segment (start 145.71 28.05) (end 131.4 28.05) (width 0.2) (layer "F.Cu") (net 11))
 (segment (start 145.92 28.26) (end 145.71 28.05) (width 0.2) (layer "F.Cu") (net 11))
 (segment (start 108.263 28.947) (end 107.14 30.07) (width 0.2) (layer "F.Cu") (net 11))
 (segment (start 131.4 28.05) (end 130.503 28.947) (width 0.2) (layer "F.Cu") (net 11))
 (segment (start 107.14 30.07) (end 109.62 32.55) (width 0.2) (layer "F.Cu") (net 11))
 (segment (start 145.92 33.19) (end 145.92 28.26) (width 0.2) (layer "F.Cu") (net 11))
 (segment (start 111.643 31.073) (end 110.58 30.01) (width 0.2) (layer "F.Cu") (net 9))
 (segment (start 129.303 31.073) (end 111.643 31.073) (width 0.2) (layer "F.Cu") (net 9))
 (segment (start 131.42 33.19) (end 129.303 31.073) (width 0.2) (layer "F.Cu") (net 9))
 (segment (start 131.42 38.19) (end 129.56692 36.33692) (width 0.2) (layer "F.Cu") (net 10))
 (segment (start 129.56692 36.33692) (end 128.99308 36.33692) (width 0.2) (layer "F.Cu") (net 10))
 (via (at 128.99308 36.33692) (size 0.6) (drill 0.3) (layers "F.Cu" "B.Cu") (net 10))
 (segment (start 128.99308 36.33692) (end 119.44692 36.33692) (width 0.2) (layer "B.Cu") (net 10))
 (segment (start 119.44692 36.33692) (end 110.58 27.47) (width 0.2) (layer "B.Cu") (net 10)))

